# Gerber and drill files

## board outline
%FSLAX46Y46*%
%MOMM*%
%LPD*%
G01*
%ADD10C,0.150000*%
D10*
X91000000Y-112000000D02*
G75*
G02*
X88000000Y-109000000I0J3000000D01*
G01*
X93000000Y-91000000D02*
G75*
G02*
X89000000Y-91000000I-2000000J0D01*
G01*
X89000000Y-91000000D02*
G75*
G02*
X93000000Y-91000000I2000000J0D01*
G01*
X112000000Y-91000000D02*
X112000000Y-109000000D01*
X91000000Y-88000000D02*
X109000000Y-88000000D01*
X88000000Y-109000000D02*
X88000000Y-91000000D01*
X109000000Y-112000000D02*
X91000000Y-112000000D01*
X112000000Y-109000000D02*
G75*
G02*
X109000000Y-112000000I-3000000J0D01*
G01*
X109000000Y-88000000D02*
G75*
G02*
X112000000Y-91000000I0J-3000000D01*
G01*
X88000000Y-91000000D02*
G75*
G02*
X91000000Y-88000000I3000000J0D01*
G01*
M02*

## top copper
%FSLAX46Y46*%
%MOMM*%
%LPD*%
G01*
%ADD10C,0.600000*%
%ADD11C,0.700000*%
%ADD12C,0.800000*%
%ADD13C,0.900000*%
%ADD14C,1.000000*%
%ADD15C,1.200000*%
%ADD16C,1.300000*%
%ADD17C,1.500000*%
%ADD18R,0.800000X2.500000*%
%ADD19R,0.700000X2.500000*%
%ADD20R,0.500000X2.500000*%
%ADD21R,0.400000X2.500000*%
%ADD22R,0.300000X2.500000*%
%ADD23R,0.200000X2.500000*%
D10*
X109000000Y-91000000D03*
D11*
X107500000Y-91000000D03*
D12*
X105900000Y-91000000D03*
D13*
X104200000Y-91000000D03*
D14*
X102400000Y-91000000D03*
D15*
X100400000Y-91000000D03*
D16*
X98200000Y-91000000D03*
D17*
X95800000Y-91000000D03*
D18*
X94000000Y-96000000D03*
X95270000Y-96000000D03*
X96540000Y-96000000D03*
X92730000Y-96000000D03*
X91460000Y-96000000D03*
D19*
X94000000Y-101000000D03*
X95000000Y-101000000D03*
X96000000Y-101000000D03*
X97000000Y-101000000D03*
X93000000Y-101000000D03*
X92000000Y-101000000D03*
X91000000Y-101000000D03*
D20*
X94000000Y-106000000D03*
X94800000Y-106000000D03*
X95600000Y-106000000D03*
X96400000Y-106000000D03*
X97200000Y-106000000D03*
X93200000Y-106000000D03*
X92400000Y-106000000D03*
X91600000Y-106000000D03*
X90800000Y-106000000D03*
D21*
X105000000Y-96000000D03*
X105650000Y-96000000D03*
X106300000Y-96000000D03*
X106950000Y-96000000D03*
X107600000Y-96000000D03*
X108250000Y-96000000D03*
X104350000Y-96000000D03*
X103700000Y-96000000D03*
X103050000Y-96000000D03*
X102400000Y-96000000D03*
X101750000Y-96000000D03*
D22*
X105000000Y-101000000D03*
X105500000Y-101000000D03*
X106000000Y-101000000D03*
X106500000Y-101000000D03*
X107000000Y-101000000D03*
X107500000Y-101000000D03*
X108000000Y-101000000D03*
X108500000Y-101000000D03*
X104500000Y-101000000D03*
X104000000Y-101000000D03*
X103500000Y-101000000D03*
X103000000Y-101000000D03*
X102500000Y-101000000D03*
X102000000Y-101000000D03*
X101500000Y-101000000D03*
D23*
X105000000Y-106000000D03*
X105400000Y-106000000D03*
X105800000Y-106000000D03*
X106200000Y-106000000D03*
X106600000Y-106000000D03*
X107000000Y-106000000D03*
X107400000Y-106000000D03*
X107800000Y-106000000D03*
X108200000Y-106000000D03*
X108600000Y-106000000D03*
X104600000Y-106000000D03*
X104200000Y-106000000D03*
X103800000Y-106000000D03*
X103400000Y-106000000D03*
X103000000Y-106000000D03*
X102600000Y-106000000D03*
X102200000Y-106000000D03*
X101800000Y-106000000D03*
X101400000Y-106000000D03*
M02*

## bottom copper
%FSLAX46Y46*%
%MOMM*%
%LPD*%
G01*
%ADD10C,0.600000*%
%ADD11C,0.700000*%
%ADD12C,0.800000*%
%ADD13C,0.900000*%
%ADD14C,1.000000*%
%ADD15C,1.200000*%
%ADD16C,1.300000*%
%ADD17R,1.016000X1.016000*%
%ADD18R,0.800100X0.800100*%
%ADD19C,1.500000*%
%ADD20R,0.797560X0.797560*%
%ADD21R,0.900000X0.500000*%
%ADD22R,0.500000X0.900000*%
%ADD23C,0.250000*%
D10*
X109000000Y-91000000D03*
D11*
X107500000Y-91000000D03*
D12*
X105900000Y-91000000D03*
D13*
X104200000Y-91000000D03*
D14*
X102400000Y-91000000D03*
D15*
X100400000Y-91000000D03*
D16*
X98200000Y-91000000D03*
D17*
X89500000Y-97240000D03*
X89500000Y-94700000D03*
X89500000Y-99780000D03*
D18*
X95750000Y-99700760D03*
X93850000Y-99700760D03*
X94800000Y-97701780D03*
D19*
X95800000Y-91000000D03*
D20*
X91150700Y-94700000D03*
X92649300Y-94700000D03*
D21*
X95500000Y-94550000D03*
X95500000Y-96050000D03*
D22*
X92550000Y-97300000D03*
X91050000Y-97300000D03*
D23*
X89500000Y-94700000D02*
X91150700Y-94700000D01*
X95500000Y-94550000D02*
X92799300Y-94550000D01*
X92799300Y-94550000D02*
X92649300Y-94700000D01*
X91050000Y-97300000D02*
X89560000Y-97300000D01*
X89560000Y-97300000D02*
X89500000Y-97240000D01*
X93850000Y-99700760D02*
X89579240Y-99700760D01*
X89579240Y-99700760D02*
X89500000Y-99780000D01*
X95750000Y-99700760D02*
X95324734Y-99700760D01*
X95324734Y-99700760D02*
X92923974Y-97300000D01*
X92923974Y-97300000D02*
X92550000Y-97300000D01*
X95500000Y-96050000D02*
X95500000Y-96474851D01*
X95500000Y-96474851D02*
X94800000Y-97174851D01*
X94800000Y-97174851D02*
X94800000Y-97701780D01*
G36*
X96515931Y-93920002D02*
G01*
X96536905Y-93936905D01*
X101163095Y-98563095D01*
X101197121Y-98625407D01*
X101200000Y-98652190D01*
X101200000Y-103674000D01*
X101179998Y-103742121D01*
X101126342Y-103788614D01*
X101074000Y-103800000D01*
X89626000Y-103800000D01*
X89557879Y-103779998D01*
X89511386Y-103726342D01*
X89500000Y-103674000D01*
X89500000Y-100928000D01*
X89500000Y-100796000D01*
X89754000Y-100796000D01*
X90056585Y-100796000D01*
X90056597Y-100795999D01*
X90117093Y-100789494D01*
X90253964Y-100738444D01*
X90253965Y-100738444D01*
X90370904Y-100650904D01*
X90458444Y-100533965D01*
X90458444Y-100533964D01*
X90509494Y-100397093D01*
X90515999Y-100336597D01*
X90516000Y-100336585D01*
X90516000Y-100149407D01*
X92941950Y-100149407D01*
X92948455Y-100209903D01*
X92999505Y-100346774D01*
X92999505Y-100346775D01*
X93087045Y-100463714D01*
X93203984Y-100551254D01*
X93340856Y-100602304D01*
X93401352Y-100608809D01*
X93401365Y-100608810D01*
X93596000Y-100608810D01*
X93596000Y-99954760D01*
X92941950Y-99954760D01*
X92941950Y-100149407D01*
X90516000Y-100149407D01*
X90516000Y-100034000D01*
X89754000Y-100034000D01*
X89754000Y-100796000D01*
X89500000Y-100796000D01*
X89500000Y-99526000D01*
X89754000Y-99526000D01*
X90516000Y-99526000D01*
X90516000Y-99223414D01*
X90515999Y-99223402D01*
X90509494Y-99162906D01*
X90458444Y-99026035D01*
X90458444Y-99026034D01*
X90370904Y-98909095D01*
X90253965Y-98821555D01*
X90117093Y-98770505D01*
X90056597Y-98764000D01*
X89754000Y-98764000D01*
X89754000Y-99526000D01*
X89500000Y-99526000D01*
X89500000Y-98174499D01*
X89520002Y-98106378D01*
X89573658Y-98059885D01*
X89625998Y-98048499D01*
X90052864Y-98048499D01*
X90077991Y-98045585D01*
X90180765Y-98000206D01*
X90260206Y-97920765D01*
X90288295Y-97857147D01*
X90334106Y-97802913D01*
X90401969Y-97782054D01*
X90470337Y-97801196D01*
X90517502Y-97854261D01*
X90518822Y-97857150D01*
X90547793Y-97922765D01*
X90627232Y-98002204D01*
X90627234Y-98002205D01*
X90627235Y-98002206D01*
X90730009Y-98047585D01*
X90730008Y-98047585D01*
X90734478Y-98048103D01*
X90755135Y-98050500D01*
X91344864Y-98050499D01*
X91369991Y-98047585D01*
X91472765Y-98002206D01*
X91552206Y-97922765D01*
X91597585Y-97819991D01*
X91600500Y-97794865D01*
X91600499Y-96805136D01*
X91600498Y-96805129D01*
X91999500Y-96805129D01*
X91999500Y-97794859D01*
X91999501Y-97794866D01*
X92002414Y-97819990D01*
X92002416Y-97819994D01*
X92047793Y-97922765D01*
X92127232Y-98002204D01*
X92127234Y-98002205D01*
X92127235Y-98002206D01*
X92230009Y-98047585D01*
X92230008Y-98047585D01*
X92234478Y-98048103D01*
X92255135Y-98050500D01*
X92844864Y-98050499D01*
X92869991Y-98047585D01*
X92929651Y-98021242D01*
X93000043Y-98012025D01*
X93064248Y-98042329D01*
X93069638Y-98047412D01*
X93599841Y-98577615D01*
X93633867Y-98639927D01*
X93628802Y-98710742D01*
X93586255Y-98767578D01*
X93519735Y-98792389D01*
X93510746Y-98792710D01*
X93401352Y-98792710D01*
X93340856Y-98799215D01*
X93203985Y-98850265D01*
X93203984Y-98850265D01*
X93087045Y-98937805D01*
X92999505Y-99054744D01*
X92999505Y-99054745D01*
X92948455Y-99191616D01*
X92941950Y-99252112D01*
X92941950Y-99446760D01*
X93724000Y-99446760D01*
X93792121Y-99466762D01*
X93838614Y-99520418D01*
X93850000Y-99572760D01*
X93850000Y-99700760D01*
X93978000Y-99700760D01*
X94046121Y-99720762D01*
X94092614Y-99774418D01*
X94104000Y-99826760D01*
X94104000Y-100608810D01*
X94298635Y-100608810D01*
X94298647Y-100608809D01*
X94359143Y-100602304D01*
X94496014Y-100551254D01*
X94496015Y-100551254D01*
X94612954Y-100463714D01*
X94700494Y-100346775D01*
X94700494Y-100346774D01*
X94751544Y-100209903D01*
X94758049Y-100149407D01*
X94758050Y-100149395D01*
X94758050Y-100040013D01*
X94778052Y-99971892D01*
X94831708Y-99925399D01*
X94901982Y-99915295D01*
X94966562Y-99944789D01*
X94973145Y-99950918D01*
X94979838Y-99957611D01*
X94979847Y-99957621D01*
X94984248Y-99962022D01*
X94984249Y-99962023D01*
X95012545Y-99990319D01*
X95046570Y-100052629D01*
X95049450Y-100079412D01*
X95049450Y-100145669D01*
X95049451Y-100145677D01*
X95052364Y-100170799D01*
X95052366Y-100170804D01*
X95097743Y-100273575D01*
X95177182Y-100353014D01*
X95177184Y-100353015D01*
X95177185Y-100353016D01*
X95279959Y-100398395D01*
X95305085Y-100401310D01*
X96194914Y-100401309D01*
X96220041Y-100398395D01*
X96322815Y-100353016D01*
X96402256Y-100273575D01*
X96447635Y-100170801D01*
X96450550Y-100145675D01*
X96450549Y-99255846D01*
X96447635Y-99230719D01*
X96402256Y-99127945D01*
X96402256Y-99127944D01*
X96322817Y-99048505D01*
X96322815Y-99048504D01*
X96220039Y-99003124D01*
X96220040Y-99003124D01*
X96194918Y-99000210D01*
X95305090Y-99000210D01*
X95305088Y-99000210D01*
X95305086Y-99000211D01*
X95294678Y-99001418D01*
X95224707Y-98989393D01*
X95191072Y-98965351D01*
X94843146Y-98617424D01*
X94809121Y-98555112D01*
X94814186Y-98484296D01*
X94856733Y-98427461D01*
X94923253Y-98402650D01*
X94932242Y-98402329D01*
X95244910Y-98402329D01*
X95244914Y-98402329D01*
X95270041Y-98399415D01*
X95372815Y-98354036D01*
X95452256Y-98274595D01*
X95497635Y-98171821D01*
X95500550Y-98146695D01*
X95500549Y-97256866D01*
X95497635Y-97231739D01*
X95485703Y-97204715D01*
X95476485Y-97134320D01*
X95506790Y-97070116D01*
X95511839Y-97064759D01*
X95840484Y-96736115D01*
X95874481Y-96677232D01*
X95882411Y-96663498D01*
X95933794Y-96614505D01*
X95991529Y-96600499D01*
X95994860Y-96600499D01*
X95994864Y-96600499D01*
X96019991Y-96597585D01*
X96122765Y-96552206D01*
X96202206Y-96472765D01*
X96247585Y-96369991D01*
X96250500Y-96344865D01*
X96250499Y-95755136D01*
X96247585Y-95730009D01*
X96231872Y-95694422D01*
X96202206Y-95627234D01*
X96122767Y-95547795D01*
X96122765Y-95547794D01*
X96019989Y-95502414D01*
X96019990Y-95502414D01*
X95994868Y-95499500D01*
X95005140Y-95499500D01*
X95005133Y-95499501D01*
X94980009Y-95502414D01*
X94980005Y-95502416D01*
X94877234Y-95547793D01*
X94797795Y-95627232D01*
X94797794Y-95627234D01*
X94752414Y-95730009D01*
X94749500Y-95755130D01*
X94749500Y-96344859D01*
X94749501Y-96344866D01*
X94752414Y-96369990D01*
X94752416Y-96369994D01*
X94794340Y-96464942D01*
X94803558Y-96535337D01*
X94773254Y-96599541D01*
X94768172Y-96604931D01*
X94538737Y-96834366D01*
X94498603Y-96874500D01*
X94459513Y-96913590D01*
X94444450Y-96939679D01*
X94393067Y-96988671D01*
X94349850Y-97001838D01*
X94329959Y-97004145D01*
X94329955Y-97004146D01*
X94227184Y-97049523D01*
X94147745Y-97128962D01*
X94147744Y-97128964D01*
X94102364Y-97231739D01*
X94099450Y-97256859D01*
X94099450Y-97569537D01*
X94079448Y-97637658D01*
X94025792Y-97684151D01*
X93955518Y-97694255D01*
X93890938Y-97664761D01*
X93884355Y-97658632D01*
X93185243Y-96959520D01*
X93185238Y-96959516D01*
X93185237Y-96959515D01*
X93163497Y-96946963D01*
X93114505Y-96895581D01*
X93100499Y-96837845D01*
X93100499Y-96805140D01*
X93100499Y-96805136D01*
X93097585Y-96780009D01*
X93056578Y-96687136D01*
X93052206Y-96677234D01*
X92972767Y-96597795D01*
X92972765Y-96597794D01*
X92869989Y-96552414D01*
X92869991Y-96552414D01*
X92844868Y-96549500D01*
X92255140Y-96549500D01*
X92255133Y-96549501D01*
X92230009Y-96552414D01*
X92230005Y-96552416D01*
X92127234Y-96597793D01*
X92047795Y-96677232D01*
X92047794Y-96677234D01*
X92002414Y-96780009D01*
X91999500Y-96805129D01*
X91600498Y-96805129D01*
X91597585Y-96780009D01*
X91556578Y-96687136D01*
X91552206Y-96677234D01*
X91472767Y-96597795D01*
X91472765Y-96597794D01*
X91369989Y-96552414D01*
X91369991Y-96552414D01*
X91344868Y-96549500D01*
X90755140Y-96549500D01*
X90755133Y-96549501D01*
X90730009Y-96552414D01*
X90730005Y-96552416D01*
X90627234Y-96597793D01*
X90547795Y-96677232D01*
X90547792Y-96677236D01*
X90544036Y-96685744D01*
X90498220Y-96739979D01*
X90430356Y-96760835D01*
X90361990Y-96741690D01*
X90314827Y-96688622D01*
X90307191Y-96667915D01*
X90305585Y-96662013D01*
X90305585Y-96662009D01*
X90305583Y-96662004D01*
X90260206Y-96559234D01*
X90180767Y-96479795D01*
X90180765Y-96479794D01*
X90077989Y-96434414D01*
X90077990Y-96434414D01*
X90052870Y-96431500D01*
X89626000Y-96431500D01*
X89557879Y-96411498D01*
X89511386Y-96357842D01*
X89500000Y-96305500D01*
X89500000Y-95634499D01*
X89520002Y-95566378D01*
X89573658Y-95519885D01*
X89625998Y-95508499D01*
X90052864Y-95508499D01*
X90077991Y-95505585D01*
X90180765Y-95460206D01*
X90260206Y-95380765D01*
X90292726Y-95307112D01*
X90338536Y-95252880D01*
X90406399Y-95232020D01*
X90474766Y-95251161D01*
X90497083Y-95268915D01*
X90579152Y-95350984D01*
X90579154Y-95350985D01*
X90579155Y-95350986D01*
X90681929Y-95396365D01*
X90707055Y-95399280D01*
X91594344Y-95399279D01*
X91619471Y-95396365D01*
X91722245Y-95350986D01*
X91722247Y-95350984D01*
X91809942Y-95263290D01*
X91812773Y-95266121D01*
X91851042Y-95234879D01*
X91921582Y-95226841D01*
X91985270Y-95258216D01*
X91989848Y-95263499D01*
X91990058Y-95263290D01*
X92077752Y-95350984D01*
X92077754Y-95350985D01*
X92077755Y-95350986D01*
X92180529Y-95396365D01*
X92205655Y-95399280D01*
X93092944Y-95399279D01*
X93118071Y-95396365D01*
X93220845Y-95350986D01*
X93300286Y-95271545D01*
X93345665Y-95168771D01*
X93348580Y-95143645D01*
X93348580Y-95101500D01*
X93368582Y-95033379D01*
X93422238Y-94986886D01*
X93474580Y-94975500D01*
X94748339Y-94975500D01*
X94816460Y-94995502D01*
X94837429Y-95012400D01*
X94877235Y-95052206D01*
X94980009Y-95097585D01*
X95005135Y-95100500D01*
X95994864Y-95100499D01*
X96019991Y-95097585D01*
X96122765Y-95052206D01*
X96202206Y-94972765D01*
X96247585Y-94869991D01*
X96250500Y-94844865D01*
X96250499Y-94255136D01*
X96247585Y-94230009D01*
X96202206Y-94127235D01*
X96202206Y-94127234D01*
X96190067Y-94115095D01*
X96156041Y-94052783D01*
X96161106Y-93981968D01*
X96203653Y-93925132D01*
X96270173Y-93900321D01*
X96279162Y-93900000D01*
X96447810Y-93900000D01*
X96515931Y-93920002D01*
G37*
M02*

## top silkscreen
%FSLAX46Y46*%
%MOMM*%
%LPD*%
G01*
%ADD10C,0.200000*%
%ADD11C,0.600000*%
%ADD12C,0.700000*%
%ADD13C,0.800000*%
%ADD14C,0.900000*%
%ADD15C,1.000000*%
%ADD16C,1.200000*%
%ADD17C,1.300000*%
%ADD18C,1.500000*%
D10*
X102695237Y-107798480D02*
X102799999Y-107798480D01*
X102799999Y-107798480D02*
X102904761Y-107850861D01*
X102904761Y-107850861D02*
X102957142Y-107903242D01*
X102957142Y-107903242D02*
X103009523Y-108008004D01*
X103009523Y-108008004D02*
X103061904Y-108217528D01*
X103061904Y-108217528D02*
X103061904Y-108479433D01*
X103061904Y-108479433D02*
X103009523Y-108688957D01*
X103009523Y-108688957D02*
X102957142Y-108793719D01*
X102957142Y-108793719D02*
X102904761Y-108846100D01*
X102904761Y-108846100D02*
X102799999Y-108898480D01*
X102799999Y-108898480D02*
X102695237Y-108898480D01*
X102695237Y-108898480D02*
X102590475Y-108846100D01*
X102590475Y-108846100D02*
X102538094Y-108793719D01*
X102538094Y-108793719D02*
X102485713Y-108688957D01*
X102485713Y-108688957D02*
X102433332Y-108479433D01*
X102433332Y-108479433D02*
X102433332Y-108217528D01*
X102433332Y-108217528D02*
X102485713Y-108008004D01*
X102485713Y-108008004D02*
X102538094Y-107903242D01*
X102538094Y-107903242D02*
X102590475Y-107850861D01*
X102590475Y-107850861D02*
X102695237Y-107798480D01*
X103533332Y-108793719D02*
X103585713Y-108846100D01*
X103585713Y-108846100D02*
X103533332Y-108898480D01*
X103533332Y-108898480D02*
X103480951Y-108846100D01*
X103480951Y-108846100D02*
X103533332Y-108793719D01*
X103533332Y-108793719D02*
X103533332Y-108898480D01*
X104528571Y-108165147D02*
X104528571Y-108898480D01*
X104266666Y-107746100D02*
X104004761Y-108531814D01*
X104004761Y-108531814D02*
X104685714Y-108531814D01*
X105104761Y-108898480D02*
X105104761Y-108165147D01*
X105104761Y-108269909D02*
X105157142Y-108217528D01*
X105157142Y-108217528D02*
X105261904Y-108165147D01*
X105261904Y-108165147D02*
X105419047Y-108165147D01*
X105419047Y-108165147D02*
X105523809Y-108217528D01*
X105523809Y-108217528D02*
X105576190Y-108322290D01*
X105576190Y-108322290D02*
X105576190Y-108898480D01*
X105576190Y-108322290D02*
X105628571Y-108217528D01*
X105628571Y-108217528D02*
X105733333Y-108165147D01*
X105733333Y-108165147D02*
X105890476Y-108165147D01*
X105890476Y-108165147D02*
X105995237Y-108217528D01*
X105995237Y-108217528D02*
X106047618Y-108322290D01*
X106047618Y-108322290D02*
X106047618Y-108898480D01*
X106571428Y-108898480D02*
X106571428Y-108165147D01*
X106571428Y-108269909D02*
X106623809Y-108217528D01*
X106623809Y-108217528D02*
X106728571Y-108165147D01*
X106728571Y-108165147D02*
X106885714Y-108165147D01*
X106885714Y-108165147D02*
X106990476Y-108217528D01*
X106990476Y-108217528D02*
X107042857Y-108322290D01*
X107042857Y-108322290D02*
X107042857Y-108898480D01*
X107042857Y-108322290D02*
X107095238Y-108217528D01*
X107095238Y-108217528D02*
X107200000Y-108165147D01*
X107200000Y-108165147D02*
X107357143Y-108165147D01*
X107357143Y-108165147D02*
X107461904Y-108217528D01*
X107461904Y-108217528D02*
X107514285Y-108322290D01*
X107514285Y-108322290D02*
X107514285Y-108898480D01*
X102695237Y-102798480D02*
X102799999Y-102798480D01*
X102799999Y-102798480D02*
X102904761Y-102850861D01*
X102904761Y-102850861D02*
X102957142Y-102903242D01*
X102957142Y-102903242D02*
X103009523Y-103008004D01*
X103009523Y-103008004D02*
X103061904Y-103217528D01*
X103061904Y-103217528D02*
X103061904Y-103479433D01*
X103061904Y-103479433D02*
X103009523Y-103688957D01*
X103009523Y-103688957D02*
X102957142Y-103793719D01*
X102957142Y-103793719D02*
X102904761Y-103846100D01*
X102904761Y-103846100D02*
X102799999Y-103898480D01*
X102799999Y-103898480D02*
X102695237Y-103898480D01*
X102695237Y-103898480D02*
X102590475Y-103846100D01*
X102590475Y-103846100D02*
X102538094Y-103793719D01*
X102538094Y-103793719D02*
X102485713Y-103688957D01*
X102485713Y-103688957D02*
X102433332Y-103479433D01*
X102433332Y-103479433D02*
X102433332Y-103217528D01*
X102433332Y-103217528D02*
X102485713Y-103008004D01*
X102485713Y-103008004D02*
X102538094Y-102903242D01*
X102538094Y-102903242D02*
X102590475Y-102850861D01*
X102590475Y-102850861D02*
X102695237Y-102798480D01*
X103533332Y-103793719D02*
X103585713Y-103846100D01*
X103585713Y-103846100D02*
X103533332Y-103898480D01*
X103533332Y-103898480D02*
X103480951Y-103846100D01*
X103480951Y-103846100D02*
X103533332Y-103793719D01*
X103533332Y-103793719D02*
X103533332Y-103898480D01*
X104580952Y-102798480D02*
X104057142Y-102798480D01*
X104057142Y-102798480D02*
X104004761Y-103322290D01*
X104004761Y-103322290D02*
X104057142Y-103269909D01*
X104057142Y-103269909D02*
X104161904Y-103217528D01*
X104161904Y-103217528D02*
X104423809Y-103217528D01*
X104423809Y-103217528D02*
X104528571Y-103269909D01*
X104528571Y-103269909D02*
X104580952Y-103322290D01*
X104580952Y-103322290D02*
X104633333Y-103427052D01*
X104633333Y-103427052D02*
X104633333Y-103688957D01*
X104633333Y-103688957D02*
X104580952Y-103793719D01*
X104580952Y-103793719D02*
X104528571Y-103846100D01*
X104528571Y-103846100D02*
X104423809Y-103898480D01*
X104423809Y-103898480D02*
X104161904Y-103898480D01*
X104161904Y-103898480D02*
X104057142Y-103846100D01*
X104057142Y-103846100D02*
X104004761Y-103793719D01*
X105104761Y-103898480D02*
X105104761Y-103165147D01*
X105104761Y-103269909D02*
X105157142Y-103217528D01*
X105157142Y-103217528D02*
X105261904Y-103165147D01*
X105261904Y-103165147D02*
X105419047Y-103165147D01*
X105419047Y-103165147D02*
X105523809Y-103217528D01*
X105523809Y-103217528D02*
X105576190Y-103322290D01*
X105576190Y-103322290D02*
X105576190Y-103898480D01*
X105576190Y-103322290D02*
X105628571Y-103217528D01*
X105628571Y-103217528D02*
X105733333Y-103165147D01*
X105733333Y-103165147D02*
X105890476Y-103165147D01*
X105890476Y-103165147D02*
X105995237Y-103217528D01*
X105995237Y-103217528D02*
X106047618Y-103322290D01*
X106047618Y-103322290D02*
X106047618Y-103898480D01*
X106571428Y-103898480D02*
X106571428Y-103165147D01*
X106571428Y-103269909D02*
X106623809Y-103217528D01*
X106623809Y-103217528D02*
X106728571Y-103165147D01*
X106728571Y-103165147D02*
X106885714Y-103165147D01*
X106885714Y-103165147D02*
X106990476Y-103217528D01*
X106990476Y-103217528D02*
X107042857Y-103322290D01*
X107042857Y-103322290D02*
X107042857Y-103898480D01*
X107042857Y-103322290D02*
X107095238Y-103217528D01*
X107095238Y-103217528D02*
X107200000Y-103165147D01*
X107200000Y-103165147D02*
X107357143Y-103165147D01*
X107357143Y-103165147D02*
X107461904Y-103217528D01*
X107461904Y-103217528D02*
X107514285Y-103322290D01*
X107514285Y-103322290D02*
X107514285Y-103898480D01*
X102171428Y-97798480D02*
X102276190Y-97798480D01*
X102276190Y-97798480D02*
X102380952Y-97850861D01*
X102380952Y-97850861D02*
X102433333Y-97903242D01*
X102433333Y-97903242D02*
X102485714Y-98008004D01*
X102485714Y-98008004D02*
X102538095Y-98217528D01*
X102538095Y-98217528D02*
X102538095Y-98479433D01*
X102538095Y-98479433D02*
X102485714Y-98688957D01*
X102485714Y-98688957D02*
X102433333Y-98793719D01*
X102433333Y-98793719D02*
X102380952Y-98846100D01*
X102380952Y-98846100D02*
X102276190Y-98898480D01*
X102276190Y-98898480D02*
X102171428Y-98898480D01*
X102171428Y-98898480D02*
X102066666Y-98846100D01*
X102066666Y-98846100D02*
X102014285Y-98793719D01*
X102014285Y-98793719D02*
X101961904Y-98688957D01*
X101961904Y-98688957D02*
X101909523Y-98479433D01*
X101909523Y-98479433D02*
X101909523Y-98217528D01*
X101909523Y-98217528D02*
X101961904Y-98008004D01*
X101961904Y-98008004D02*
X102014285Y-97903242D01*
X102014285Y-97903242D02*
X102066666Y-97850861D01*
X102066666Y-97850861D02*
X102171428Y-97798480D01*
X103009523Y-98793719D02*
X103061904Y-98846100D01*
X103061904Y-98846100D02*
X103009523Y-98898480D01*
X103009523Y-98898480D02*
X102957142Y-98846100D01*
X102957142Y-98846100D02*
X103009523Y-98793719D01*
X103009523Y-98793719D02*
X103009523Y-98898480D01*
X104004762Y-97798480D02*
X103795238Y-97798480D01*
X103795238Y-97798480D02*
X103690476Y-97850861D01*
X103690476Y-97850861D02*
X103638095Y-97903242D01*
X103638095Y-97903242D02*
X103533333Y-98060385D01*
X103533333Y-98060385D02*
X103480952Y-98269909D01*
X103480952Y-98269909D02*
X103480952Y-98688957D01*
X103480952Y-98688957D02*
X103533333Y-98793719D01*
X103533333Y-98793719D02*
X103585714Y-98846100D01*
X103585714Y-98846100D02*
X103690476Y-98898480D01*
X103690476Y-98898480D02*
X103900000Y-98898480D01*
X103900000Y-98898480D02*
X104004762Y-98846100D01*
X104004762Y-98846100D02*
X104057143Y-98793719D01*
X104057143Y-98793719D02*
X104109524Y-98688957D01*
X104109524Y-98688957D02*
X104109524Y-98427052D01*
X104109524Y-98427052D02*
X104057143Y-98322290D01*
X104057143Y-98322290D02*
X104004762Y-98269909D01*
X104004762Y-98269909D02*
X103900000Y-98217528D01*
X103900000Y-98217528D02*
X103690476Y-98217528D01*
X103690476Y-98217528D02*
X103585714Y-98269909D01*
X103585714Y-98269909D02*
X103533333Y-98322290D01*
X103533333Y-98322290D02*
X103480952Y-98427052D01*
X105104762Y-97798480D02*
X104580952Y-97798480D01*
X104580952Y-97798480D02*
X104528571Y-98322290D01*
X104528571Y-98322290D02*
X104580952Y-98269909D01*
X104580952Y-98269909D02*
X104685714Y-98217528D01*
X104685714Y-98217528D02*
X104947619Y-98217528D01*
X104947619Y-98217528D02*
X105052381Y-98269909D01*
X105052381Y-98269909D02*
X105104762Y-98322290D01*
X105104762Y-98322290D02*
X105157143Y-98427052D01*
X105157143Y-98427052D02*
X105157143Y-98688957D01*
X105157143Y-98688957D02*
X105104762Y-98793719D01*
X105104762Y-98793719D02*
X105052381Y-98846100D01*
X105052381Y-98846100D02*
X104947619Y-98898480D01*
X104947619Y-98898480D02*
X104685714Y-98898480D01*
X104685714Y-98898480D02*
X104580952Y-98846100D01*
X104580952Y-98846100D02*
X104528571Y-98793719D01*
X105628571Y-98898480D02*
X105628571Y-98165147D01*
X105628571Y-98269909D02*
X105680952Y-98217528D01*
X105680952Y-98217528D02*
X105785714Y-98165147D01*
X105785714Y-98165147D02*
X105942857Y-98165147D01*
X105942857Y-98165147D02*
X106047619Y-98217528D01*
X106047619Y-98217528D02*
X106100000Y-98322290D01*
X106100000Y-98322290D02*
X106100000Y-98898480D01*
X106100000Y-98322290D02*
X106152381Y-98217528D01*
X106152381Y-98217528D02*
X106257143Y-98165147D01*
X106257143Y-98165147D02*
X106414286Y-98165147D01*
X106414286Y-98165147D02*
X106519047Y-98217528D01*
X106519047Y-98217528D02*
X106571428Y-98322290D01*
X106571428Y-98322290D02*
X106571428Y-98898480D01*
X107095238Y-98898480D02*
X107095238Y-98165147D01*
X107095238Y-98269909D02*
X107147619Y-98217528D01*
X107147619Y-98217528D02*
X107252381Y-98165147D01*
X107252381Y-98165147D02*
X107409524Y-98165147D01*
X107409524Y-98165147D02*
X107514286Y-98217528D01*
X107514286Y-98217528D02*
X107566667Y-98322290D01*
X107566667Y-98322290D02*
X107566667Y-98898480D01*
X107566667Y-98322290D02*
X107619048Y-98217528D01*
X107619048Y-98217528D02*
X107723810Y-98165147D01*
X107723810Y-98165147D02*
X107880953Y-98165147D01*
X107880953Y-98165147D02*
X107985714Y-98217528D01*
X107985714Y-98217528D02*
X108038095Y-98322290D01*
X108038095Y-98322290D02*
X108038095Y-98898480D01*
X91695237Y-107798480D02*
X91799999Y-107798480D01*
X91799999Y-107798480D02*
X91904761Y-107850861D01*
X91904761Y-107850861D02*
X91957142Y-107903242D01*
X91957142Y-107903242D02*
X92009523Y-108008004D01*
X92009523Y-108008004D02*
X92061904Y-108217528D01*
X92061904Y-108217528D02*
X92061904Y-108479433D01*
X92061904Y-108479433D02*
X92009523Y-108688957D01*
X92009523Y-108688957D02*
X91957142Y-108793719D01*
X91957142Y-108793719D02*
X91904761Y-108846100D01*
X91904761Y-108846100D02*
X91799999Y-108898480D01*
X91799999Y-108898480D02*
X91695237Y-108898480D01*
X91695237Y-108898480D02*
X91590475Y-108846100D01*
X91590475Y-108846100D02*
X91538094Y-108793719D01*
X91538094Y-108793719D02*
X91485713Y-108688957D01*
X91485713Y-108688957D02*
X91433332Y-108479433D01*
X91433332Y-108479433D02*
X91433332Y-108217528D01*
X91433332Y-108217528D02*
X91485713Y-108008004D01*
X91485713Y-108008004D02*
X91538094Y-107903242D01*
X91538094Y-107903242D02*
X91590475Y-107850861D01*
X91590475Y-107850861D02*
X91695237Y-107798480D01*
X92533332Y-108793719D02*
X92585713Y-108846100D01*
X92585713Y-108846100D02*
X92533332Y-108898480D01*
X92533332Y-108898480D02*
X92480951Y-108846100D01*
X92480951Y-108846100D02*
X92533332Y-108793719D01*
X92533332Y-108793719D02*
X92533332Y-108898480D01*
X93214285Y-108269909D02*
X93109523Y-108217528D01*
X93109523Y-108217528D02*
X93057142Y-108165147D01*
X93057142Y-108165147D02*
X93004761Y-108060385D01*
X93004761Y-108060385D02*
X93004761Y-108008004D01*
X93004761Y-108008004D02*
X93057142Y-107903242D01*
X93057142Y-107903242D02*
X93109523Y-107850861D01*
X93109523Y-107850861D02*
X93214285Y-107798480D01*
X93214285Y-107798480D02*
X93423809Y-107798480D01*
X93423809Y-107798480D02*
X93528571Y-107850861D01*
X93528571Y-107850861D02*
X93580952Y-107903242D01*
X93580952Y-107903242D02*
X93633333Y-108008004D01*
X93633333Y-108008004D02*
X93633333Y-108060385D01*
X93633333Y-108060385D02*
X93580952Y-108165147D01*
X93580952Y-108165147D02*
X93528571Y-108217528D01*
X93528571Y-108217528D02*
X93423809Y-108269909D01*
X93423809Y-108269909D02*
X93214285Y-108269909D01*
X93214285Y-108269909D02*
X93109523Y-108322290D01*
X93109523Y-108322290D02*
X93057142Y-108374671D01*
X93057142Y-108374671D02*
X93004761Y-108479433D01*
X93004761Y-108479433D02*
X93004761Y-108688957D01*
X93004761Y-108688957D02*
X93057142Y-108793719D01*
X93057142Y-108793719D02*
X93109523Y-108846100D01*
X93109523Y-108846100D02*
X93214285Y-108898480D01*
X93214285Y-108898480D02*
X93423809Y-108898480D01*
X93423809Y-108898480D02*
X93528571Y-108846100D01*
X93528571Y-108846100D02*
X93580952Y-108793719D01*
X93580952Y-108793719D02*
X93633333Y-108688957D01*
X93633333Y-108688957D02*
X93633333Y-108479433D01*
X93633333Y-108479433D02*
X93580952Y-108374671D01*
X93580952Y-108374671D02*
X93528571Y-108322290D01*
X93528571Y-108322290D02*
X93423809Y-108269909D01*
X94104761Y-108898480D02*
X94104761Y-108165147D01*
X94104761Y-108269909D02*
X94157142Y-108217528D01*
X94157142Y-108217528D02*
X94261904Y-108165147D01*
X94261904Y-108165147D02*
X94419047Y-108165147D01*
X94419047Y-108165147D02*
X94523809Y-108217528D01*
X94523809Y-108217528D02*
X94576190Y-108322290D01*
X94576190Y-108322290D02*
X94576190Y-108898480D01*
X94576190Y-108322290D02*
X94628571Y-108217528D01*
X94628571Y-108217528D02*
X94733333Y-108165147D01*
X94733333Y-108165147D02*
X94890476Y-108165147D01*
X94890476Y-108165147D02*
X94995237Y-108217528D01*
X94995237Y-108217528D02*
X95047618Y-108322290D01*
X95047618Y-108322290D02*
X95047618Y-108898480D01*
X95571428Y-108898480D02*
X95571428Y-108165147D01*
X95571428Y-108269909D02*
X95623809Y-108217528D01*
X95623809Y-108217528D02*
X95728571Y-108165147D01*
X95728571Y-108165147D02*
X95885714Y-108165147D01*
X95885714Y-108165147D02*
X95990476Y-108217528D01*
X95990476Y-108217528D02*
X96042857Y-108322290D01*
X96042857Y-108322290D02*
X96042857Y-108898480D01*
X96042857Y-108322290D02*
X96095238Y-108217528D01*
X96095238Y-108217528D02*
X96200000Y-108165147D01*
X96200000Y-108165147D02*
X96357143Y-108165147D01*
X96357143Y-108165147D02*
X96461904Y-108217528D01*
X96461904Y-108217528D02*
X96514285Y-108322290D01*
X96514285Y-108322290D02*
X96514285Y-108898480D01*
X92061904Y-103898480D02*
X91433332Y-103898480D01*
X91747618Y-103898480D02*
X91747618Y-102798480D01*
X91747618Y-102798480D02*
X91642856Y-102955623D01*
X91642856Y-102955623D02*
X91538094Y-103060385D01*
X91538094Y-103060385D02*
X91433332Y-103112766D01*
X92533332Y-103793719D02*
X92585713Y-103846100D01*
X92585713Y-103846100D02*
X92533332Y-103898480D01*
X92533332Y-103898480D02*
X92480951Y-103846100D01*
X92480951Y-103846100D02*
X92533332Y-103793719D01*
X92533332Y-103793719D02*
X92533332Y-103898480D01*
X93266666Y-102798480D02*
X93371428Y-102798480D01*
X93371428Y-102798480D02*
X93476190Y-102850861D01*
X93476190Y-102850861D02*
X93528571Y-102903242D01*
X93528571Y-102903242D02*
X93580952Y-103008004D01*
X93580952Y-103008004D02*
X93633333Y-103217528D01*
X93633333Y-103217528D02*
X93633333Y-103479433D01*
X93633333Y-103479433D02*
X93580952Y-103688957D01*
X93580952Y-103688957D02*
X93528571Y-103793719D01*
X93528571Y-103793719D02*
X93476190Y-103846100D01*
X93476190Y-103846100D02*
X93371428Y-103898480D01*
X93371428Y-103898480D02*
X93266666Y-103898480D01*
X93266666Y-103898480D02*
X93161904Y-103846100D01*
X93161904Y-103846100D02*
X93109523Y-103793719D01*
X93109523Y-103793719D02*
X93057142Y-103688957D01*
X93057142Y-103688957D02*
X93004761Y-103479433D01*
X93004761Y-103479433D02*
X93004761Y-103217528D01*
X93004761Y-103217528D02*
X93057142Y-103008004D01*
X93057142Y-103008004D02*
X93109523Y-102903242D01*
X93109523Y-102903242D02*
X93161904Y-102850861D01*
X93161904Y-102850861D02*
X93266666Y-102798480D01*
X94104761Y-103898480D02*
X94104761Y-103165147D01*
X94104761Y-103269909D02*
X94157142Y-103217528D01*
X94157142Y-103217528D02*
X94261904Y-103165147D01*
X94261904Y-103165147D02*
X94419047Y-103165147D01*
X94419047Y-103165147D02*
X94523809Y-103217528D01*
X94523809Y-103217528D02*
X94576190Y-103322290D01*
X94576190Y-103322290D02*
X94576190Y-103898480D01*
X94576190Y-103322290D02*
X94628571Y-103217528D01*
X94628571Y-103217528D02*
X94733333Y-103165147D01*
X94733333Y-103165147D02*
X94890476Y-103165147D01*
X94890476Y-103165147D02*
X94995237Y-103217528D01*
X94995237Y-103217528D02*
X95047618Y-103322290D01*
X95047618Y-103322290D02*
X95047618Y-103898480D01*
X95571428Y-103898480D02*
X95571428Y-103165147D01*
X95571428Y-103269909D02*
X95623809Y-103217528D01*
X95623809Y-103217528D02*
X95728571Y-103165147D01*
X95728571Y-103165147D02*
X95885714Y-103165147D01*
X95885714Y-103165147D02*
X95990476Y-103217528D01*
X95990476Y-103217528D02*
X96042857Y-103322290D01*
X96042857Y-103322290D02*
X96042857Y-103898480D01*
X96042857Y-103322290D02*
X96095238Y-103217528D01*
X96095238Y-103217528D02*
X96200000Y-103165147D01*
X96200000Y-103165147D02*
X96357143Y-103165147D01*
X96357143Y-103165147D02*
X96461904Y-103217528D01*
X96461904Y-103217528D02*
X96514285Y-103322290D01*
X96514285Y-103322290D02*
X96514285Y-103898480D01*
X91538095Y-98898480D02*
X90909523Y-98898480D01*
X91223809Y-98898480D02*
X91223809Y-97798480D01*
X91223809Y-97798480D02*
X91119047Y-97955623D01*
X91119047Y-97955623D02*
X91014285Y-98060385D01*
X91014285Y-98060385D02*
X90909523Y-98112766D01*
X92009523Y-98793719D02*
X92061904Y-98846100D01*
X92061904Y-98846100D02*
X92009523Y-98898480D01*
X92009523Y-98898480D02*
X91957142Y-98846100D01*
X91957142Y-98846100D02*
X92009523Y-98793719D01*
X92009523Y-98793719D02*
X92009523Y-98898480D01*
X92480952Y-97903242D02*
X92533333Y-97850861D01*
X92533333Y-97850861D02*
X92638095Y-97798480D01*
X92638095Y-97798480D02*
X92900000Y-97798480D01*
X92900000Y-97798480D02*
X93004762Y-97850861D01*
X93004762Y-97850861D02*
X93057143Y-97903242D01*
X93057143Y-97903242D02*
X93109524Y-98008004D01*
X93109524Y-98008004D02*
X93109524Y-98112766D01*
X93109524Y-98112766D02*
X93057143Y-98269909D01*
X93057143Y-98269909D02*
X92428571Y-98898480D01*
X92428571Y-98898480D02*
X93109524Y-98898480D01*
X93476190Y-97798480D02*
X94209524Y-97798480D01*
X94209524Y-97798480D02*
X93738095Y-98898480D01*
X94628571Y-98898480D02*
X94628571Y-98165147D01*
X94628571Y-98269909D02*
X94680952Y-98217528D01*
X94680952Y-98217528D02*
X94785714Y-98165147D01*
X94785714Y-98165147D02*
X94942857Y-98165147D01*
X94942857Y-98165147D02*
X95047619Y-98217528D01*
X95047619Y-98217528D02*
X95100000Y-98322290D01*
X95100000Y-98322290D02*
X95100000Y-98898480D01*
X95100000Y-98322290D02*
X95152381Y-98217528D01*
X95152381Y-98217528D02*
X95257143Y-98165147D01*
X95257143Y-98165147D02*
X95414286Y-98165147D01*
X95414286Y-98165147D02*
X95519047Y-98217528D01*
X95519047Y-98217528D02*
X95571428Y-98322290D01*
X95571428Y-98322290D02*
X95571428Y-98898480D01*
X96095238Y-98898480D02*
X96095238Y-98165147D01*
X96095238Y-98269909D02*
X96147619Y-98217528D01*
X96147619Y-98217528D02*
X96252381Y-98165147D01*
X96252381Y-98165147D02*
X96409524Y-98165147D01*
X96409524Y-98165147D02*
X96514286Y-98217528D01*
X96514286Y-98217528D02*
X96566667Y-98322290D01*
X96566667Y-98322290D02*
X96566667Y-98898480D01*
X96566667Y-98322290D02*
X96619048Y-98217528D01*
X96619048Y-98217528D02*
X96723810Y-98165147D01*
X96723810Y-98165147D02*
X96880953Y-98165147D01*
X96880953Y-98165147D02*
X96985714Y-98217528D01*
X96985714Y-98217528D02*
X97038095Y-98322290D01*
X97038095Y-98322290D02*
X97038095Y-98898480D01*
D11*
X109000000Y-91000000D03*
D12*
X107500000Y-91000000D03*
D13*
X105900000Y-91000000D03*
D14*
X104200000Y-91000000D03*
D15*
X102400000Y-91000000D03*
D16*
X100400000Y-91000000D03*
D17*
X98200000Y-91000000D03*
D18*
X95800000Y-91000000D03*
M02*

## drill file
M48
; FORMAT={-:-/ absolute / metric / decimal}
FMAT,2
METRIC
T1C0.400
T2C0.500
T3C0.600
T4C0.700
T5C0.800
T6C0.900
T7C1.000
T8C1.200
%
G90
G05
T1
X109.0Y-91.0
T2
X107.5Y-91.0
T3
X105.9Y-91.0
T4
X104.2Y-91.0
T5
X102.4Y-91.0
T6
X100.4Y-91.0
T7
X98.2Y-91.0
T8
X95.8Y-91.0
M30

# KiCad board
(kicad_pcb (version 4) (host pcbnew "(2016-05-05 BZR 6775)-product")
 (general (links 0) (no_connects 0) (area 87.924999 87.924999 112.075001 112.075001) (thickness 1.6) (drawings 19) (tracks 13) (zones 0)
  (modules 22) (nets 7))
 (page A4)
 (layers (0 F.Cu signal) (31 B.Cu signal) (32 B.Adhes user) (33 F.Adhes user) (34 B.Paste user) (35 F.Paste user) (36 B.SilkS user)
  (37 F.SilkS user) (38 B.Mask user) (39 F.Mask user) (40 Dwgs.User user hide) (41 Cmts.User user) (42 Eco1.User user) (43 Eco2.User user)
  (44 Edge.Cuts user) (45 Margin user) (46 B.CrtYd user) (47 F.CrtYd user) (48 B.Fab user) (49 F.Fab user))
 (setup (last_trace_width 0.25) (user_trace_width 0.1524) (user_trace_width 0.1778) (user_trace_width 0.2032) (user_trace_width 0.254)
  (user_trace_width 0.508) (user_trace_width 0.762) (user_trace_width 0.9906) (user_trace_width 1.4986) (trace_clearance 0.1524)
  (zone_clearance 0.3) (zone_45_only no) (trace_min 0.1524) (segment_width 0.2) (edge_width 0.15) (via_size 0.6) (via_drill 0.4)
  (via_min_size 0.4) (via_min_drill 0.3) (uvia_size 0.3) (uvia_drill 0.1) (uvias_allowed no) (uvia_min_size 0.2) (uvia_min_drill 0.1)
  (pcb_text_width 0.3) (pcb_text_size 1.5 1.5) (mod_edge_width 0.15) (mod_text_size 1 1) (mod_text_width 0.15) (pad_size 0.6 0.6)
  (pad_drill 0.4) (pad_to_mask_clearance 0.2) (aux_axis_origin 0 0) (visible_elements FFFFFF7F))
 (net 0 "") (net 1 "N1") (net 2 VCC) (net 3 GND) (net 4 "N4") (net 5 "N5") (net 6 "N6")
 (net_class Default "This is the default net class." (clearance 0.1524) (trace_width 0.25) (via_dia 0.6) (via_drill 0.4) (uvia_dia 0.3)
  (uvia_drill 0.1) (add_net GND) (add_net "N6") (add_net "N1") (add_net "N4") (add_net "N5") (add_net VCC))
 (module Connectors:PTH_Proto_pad (layer F.Cu) (at 109 91)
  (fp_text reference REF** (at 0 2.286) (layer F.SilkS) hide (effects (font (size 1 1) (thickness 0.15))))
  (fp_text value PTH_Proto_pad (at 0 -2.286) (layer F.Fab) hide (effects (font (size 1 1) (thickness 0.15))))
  (pad 1 thru_hole circle (at 0 0) (size 0.6 0.6) (drill 0.4) (layers *.Cu *.Mask F.SilkS)))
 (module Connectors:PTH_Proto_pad (layer F.Cu) (at 107.5 91)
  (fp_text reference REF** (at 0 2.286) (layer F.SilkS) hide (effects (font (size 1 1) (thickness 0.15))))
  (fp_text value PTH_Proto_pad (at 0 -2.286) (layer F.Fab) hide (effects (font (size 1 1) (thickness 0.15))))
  (pad 1 thru_hole circle (at 0 0) (size 0.7 0.7) (drill 0.5) (layers *.Cu *.Mask F.SilkS)))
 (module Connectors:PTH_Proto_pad (layer F.Cu) (at 105.9 91)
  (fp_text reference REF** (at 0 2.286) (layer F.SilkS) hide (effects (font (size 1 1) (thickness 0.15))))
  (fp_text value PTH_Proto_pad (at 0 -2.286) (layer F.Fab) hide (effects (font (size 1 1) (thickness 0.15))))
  (pad 1 thru_hole circle (at 0 0) (size 0.8 0.8) (drill 0.6) (layers *.Cu *.Mask F.SilkS)))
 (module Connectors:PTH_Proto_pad (layer F.Cu) (at 104.2 91)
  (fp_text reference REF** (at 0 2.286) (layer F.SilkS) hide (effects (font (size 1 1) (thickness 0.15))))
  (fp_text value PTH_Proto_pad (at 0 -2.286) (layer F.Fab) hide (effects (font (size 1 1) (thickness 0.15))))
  (pad 1 thru_hole circle (at 0 0) (size 0.9 0.9) (drill 0.7) (layers *.Cu *.Mask F.SilkS)))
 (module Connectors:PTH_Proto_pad (layer F.Cu) (at 102.4 91)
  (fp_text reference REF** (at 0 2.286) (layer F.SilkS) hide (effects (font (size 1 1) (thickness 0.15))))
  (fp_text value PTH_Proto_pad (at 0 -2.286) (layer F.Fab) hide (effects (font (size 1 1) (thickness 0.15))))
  (pad 1 thru_hole circle (at 0 0) (size 1 1) (drill 0.8) (layers *.Cu *.Mask F.SilkS)))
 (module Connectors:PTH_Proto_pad (layer F.Cu) (at 100.4 91)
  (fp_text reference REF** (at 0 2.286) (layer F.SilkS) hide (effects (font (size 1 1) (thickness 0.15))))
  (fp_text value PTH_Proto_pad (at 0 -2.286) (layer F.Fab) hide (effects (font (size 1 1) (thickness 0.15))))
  (pad 1 thru_hole circle (at 0 0) (size 1.2 1.2) (drill 0.9) (layers *.Cu *.Mask F.SilkS)))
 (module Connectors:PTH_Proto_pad (layer F.Cu) (at 98.2 91)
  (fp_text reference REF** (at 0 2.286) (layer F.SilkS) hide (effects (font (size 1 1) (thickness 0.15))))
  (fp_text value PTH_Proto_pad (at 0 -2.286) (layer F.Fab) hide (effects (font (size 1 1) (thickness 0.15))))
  (pad 1 thru_hole circle (at 0 0) (size 1.3 1.3) (drill 1) (layers *.Cu *.Mask F.SilkS)))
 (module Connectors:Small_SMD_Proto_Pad (layer B.Cu) (at 89.5 97.24)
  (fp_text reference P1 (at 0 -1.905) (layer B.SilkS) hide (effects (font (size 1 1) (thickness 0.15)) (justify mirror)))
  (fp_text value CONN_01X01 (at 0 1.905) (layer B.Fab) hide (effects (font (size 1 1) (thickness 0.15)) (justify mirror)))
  (pad 1 smd rect (at 0 0) (size 1.016 1.016) (layers B.Cu B.Paste B.Mask) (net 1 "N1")))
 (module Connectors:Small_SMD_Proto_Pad (layer B.Cu) (at 89.5 94.7)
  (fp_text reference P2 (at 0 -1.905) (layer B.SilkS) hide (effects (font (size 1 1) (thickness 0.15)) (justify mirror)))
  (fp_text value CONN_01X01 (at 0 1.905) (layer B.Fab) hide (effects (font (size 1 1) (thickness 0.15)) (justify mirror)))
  (pad 1 smd rect (at 0 0) (size 1.016 1.016) (layers B.Cu B.Paste B.Mask) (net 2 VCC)))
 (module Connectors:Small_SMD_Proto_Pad (layer B.Cu) (at 89.5 99.78)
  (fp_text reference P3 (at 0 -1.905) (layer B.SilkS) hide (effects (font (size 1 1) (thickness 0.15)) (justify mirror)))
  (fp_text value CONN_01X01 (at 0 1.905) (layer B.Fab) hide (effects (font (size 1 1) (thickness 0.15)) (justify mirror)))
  (pad 1 smd rect (at 0 0) (size 1.016 1.016) (layers B.Cu B.Paste B.Mask) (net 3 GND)))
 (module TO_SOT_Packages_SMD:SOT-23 (layer B.Cu) (at 94.8 98.7 180)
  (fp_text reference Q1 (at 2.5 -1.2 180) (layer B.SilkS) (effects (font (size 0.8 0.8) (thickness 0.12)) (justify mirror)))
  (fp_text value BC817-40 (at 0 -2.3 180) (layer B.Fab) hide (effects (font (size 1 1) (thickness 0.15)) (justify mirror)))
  (pad 1 smd rect (at -0.95 -1.00076 180) (size 0.8001 0.8001) (layers B.Cu B.Paste B.Mask) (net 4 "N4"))
  (pad 2 smd rect (at 0.95 -1.00076 180) (size 0.8001 0.8001) (layers B.Cu B.Paste B.Mask) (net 3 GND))
  (pad 3 smd rect (at 0 0.99822 180) (size 0.8001 0.8001) (layers B.Cu B.Paste B.Mask) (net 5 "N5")))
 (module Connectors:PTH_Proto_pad (layer F.Cu) (at 95.8 91)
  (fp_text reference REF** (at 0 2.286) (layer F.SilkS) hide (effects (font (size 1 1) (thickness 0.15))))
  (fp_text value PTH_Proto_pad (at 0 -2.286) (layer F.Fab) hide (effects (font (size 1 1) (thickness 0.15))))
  (pad 1 thru_hole circle (at 0 0) (size 1.5 1.5) (drill 1.2) (layers *.Cu *.Mask F.SilkS)))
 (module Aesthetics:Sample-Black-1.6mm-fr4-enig (layer B.Cu) (at 100 102.6 180)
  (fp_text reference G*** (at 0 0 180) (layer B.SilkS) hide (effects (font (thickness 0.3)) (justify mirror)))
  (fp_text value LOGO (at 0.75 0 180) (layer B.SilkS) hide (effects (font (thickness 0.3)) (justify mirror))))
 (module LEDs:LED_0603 (layer B.Cu) (at 91.9 94.7 180)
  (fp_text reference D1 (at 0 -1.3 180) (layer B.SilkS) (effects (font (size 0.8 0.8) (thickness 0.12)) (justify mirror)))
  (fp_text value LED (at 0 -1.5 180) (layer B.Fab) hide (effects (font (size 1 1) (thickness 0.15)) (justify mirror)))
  (pad 2 smd rect (at 0.7493 0) (size 0.79756 0.79756) (layers B.Cu B.Paste B.Mask) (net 2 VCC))
  (pad 1 smd rect (at -0.7493 0) (size 0.79756 0.79756) (layers B.Cu B.Paste B.Mask) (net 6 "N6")))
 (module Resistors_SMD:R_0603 (layer B.Cu) (at 95.5 95.3 270)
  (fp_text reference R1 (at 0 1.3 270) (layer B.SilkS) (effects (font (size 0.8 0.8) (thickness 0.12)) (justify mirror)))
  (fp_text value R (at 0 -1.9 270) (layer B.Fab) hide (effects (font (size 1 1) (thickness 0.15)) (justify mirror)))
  (pad 1 smd rect (at -0.75 0 270) (size 0.5 0.9) (layers B.Cu B.Paste B.Mask) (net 6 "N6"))
  (pad 2 smd rect (at 0.75 0 270) (size 0.5 0.9) (layers B.Cu B.Paste B.Mask) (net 5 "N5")))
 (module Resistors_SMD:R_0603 (layer B.Cu) (at 91.8 97.3 180)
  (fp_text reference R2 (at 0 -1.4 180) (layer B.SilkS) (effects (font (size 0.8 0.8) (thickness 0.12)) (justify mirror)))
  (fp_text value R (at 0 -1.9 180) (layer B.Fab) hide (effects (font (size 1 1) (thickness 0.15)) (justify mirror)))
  (pad 1 smd rect (at -0.75 0 180) (size 0.5 0.9) (layers B.Cu B.Paste B.Mask) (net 4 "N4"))
  (pad 2 smd rect (at 0.75 0 180) (size 0.5 0.9) (layers B.Cu B.Paste B.Mask) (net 1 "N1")))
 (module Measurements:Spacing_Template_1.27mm (layer F.Cu) (at 94 96)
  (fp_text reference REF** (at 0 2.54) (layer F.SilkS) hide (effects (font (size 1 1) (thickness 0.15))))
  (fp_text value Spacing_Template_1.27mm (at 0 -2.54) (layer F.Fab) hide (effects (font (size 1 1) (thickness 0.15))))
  (pad 1 smd rect (at 0 0) (size 0.8 2.5) (layers F.Cu F.Paste F.Mask))
  (pad 1 smd rect (at 1.27 0) (size 0.8 2.5) (layers F.Cu F.Paste F.Mask))
  (pad 1 smd rect (at 2.54 0) (size 0.8 2.5) (layers F.Cu F.Paste F.Mask))
  (pad 1 smd rect (at -1.27 0) (size 0.8 2.5) (layers F.Cu F.Paste F.Mask))
  (pad 1 smd rect (at -2.54 0) (size 0.8 2.5) (layers F.Cu F.Paste F.Mask)))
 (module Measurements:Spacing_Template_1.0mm (layer F.Cu) (at 94 101)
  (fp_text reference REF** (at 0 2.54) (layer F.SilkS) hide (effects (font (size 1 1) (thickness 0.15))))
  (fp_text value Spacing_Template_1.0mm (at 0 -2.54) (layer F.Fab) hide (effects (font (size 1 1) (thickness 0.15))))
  (pad 1 smd rect (at 0 0) (size 0.7 2.5) (layers F.Cu F.Paste F.Mask))
  (pad 1 smd rect (at 1 0) (size 0.7 2.5) (layers F.Cu F.Paste F.Mask))
  (pad 1 smd rect (at 2 0) (size 0.7 2.5) (layers F.Cu F.Paste F.Mask))
  (pad 1 smd rect (at 3 0) (size 0.7 2.5) (layers F.Cu F.Paste F.Mask))
  (pad 1 smd rect (at -1 0) (size 0.7 2.5) (layers F.Cu F.Paste F.Mask))
  (pad 1 smd rect (at -2 0) (size 0.7 2.5) (layers F.Cu F.Paste F.Mask))
  (pad 1 smd rect (at -3 0) (size 0.7 2.5) (layers F.Cu F.Paste F.Mask)))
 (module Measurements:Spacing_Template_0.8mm (layer F.Cu) (at 94 106)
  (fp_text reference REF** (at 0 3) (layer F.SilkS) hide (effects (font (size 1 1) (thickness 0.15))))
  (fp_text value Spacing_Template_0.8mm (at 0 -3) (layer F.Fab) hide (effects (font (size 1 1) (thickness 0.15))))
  (pad 1 smd rect (at 0 0) (size 0.5 2.5) (layers F.Cu F.Paste F.Mask))
  (pad 1 smd rect (at 0.8 0) (size 0.5 2.5) (layers F.Cu F.Paste F.Mask))
  (pad 1 smd rect (at 1.6 0) (size 0.5 2.5) (layers F.Cu F.Paste F.Mask))
  (pad 1 smd rect (at 2.4 0) (size 0.5 2.5) (layers F.Cu F.Paste F.Mask))
  (pad 1 smd rect (at 3.2 0) (size 0.5 2.5) (layers F.Cu F.Paste F.Mask))
  (pad 1 smd rect (at -0.8 0) (size 0.5 2.5) (layers F.Cu F.Paste F.Mask))
  (pad 1 smd rect (at -1.6 0) (size 0.5 2.5) (layers F.Cu F.Paste F.Mask))
  (pad 1 smd rect (at -2.4 0) (size 0.5 2.5) (layers F.Cu F.Paste F.Mask))
  (pad 1 smd rect (at -3.2 0) (size 0.5 2.5) (layers F.Cu F.Paste F.Mask)))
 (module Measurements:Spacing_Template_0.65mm (layer F.Cu) (at 105 96)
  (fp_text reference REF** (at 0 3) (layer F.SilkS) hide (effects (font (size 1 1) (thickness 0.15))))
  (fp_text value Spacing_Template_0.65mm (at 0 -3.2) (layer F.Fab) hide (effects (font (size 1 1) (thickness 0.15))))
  (pad 1 smd rect (at 0 0) (size 0.4 2.5) (layers F.Cu F.Paste F.Mask))
  (pad 1 smd rect (at 0.65 0) (size 0.4 2.5) (layers F.Cu F.Paste F.Mask))
  (pad 1 smd rect (at 1.3 0) (size 0.4 2.5) (layers F.Cu F.Paste F.Mask))
  (pad 1 smd rect (at 1.95 0) (size 0.4 2.5) (layers F.Cu F.Paste F.Mask))
  (pad 1 smd rect (at 2.6 0) (size 0.4 2.5) (layers F.Cu F.Paste F.Mask))
  (pad 1 smd rect (at 3.25 0) (size 0.4 2.5) (layers F.Cu F.Paste F.Mask))
  (pad 1 smd rect (at -0.65 0) (size 0.4 2.5) (layers F.Cu F.Paste F.Mask))
  (pad 1 smd rect (at -1.3 0) (size 0.4 2.5) (layers F.Cu F.Paste F.Mask))
  (pad 1 smd rect (at -1.95 0) (size 0.4 2.5) (layers F.Cu F.Paste F.Mask))
  (pad 1 smd rect (at -2.6 0) (size 0.4 2.5) (layers F.Cu F.Paste F.Mask))
  (pad 1 smd rect (at -3.25 0) (size 0.4 2.5) (layers F.Cu F.Paste F.Mask)))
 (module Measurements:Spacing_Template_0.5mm (layer F.Cu) (at 105 101)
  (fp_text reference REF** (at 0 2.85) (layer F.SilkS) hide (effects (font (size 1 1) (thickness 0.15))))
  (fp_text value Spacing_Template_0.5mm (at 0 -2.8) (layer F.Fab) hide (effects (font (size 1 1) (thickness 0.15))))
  (pad 1 smd rect (at 0 0) (size 0.3 2.5) (layers F.Cu F.Paste F.Mask))
  (pad 1 smd rect (at 0.5 0) (size 0.3 2.5) (layers F.Cu F.Paste F.Mask))
  (pad 1 smd rect (at 1 0) (size 0.3 2.5) (layers F.Cu F.Paste F.Mask))
  (pad 1 smd rect (at 1.5 0) (size 0.3 2.5) (layers F.Cu F.Paste F.Mask))
  (pad 1 smd rect (at 2 0) (size 0.3 2.5) (layers F.Cu F.Paste F.Mask))
  (pad 1 smd rect (at 2.5 0) (size 0.3 2.5) (layers F.Cu F.Paste F.Mask))
  (pad 1 smd rect (at 3 0) (size 0.3 2.5) (layers F.Cu F.Paste F.Mask))
  (pad 1 smd rect (at 3.5 0) (size 0.3 2.5) (layers F.Cu F.Paste F.Mask))
  (pad 1 smd rect (at -0.5 0) (size 0.3 2.5) (layers F.Cu F.Paste F.Mask))
  (pad 1 smd rect (at -1 0) (size 0.3 2.5) (layers F.Cu F.Paste F.Mask))
  (pad 1 smd rect (at -1.5 0) (size 0.3 2.5) (layers F.Cu F.Paste F.Mask))
  (pad 1 smd rect (at -2 0) (size 0.3 2.5) (layers F.Cu F.Paste F.Mask))
  (pad 1 smd rect (at -2.5 0) (size 0.3 2.5) (layers F.Cu F.Paste F.Mask))
  (pad 1 smd rect (at -3 0) (size 0.3 2.5) (layers F.Cu F.Paste F.Mask))
  (pad 1 smd rect (at -3.5 0) (size 0.3 2.5) (layers F.Cu F.Paste F.Mask)))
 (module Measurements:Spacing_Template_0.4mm (layer F.Cu) (at 105 106)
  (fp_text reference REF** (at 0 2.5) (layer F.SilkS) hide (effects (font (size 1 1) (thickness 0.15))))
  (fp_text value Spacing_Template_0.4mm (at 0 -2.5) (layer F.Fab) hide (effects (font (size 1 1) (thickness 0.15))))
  (pad 1 smd rect (at 0 0) (size 0.2 2.5) (layers F.Cu F.Paste F.Mask))
  (pad 1 smd rect (at 0.4 0) (size 0.2 2.5) (layers F.Cu F.Paste F.Mask))
  (pad 1 smd rect (at 0.8 0) (size 0.2 2.5) (layers F.Cu F.Paste F.Mask))
  (pad 1 smd rect (at 1.2 0) (size 0.2 2.5) (layers F.Cu F.Paste F.Mask))
  (pad 1 smd rect (at 1.6 0) (size 0.2 2.5) (layers F.Cu F.Paste F.Mask))
  (pad 1 smd rect (at 2 0) (size 0.2 2.5) (layers F.Cu F.Paste F.Mask))
  (pad 1 smd rect (at 2.4 0) (size 0.2 2.5) (layers F.Cu F.Paste F.Mask))
  (pad 1 smd rect (at 2.8 0) (size 0.2 2.5) (layers F.Cu F.Paste F.Mask))
  (pad 1 smd rect (at 3.2 0) (size 0.2 2.5) (layers F.Cu F.Paste F.Mask))
  (pad 1 smd rect (at 3.6 0) (size 0.2 2.5) (layers F.Cu F.Paste F.Mask))
  (pad 1 smd rect (at -0.4 0) (size 0.2 2.5) (layers F.Cu F.Paste F.Mask))
  (pad 1 smd rect (at -0.8 0) (size 0.2 2.5) (layers F.Cu F.Paste F.Mask))
  (pad 1 smd rect (at -1.2 0) (size 0.2 2.5) (layers F.Cu F.Paste F.Mask))
  (pad 1 smd rect (at -1.6 0) (size 0.2 2.5) (layers F.Cu F.Paste F.Mask))
  (pad 1 smd rect (at -2 0) (size 0.2 2.5) (layers F.Cu F.Paste F.Mask))
  (pad 1 smd rect (at -2.4 0) (size 0.2 2.5) (layers F.Cu F.Paste F.Mask))
  (pad 1 smd rect (at -2.8 0) (size 0.2 2.5) (layers F.Cu F.Paste F.Mask))
  (pad 1 smd rect (at -3.2 0) (size 0.2 2.5) (layers F.Cu F.Paste F.Mask))
  (pad 1 smd rect (at -3.6 0) (size 0.2 2.5) (layers F.Cu F.Paste F.Mask)))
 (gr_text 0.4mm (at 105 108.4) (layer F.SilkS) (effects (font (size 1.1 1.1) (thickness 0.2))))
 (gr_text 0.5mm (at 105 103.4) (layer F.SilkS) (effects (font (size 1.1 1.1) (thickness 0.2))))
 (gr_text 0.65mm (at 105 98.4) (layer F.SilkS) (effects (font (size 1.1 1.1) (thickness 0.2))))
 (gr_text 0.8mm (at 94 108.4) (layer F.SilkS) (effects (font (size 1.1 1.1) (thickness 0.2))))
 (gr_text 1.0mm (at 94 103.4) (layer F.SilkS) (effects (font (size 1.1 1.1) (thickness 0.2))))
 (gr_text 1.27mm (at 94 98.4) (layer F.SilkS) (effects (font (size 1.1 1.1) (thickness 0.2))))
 (gr_arc (start 91 109) (end 91 112) (angle 90) (layer Edge.Cuts) (width 0.15))
 (gr_circle (center 91 91) (end 93 91) (layer Edge.Cuts) (width 0.15))
 (gr_line (start 112 91) (end 112 109) (layer Edge.Cuts) (width 0.15))
 (gr_line (start 91 88) (end 109 88) (layer Edge.Cuts) (width 0.15))
 (gr_line (start 88 109) (end 88 91) (layer Edge.Cuts) (width 0.15))
 (gr_line (start 109 112) (end 91 112) (layer Edge.Cuts) (width 0.15))
 (gr_arc (start 109 109) (end 112 109) (angle 90) (layer Edge.Cuts) (width 0.15))
 (gr_arc (start 109 91) (end 109 88) (angle 90) (layer Edge.Cuts) (width 0.15))
 (gr_arc (start 91 91) (end 88 91) (angle 90) (layer Edge.Cuts) (width 0.15))
 (segment (start 89.5 94.7) (end 91.1507 94.7) (width 0.25) (layer B.Cu) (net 2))
 (segment (start 95.5 94.55) (end 92.7993 94.55) (width 0.25) (layer B.Cu) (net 6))
 (segment (start 92.7993 94.55) (end 92.6493 94.7) (width 0.25) (layer B.Cu) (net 6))
 (segment (start 91.05 97.3) (end 89.56 97.3) (width 0.25) (layer B.Cu) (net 1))
 (segment (start 89.56 97.3) (end 89.5 97.24) (width 0.25) (layer B.Cu) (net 1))
 (segment (start 93.85 99.70076) (end 89.57924 99.70076) (width 0.25) (layer B.Cu) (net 3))
 (segment (start 89.57924 99.70076) (end 89.5 99.78) (width 0.25) (layer B.Cu) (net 3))
 (segment (start 95.75 99.70076) (end 95.324734 99.70076) (width 0.25) (layer B.Cu) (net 4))
 (segment (start 95.324734 99.70076) (end 92.923974 97.3) (width 0.25) (layer B.Cu) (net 4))
 (segment (start 92.923974 97.3) (end 92.55 97.3) (width 0.25) (layer B.Cu) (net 4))
 (segment (start 95.5 96.05) (end 95.5 96.474851) (width 0.25) (layer B.Cu) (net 5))
 (segment (start 95.5 96.474851) (end 94.8 97.174851) (width 0.25) (layer B.Cu) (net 5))
 (segment (start 94.8 97.174851) (end 94.8 97.70178) (width 0.25) (layer B.Cu) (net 5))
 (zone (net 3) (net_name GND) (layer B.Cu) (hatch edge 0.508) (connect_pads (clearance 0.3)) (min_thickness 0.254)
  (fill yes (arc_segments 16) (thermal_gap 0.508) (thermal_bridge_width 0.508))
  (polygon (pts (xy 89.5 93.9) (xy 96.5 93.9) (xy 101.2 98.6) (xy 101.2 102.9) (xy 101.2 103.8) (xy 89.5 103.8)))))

